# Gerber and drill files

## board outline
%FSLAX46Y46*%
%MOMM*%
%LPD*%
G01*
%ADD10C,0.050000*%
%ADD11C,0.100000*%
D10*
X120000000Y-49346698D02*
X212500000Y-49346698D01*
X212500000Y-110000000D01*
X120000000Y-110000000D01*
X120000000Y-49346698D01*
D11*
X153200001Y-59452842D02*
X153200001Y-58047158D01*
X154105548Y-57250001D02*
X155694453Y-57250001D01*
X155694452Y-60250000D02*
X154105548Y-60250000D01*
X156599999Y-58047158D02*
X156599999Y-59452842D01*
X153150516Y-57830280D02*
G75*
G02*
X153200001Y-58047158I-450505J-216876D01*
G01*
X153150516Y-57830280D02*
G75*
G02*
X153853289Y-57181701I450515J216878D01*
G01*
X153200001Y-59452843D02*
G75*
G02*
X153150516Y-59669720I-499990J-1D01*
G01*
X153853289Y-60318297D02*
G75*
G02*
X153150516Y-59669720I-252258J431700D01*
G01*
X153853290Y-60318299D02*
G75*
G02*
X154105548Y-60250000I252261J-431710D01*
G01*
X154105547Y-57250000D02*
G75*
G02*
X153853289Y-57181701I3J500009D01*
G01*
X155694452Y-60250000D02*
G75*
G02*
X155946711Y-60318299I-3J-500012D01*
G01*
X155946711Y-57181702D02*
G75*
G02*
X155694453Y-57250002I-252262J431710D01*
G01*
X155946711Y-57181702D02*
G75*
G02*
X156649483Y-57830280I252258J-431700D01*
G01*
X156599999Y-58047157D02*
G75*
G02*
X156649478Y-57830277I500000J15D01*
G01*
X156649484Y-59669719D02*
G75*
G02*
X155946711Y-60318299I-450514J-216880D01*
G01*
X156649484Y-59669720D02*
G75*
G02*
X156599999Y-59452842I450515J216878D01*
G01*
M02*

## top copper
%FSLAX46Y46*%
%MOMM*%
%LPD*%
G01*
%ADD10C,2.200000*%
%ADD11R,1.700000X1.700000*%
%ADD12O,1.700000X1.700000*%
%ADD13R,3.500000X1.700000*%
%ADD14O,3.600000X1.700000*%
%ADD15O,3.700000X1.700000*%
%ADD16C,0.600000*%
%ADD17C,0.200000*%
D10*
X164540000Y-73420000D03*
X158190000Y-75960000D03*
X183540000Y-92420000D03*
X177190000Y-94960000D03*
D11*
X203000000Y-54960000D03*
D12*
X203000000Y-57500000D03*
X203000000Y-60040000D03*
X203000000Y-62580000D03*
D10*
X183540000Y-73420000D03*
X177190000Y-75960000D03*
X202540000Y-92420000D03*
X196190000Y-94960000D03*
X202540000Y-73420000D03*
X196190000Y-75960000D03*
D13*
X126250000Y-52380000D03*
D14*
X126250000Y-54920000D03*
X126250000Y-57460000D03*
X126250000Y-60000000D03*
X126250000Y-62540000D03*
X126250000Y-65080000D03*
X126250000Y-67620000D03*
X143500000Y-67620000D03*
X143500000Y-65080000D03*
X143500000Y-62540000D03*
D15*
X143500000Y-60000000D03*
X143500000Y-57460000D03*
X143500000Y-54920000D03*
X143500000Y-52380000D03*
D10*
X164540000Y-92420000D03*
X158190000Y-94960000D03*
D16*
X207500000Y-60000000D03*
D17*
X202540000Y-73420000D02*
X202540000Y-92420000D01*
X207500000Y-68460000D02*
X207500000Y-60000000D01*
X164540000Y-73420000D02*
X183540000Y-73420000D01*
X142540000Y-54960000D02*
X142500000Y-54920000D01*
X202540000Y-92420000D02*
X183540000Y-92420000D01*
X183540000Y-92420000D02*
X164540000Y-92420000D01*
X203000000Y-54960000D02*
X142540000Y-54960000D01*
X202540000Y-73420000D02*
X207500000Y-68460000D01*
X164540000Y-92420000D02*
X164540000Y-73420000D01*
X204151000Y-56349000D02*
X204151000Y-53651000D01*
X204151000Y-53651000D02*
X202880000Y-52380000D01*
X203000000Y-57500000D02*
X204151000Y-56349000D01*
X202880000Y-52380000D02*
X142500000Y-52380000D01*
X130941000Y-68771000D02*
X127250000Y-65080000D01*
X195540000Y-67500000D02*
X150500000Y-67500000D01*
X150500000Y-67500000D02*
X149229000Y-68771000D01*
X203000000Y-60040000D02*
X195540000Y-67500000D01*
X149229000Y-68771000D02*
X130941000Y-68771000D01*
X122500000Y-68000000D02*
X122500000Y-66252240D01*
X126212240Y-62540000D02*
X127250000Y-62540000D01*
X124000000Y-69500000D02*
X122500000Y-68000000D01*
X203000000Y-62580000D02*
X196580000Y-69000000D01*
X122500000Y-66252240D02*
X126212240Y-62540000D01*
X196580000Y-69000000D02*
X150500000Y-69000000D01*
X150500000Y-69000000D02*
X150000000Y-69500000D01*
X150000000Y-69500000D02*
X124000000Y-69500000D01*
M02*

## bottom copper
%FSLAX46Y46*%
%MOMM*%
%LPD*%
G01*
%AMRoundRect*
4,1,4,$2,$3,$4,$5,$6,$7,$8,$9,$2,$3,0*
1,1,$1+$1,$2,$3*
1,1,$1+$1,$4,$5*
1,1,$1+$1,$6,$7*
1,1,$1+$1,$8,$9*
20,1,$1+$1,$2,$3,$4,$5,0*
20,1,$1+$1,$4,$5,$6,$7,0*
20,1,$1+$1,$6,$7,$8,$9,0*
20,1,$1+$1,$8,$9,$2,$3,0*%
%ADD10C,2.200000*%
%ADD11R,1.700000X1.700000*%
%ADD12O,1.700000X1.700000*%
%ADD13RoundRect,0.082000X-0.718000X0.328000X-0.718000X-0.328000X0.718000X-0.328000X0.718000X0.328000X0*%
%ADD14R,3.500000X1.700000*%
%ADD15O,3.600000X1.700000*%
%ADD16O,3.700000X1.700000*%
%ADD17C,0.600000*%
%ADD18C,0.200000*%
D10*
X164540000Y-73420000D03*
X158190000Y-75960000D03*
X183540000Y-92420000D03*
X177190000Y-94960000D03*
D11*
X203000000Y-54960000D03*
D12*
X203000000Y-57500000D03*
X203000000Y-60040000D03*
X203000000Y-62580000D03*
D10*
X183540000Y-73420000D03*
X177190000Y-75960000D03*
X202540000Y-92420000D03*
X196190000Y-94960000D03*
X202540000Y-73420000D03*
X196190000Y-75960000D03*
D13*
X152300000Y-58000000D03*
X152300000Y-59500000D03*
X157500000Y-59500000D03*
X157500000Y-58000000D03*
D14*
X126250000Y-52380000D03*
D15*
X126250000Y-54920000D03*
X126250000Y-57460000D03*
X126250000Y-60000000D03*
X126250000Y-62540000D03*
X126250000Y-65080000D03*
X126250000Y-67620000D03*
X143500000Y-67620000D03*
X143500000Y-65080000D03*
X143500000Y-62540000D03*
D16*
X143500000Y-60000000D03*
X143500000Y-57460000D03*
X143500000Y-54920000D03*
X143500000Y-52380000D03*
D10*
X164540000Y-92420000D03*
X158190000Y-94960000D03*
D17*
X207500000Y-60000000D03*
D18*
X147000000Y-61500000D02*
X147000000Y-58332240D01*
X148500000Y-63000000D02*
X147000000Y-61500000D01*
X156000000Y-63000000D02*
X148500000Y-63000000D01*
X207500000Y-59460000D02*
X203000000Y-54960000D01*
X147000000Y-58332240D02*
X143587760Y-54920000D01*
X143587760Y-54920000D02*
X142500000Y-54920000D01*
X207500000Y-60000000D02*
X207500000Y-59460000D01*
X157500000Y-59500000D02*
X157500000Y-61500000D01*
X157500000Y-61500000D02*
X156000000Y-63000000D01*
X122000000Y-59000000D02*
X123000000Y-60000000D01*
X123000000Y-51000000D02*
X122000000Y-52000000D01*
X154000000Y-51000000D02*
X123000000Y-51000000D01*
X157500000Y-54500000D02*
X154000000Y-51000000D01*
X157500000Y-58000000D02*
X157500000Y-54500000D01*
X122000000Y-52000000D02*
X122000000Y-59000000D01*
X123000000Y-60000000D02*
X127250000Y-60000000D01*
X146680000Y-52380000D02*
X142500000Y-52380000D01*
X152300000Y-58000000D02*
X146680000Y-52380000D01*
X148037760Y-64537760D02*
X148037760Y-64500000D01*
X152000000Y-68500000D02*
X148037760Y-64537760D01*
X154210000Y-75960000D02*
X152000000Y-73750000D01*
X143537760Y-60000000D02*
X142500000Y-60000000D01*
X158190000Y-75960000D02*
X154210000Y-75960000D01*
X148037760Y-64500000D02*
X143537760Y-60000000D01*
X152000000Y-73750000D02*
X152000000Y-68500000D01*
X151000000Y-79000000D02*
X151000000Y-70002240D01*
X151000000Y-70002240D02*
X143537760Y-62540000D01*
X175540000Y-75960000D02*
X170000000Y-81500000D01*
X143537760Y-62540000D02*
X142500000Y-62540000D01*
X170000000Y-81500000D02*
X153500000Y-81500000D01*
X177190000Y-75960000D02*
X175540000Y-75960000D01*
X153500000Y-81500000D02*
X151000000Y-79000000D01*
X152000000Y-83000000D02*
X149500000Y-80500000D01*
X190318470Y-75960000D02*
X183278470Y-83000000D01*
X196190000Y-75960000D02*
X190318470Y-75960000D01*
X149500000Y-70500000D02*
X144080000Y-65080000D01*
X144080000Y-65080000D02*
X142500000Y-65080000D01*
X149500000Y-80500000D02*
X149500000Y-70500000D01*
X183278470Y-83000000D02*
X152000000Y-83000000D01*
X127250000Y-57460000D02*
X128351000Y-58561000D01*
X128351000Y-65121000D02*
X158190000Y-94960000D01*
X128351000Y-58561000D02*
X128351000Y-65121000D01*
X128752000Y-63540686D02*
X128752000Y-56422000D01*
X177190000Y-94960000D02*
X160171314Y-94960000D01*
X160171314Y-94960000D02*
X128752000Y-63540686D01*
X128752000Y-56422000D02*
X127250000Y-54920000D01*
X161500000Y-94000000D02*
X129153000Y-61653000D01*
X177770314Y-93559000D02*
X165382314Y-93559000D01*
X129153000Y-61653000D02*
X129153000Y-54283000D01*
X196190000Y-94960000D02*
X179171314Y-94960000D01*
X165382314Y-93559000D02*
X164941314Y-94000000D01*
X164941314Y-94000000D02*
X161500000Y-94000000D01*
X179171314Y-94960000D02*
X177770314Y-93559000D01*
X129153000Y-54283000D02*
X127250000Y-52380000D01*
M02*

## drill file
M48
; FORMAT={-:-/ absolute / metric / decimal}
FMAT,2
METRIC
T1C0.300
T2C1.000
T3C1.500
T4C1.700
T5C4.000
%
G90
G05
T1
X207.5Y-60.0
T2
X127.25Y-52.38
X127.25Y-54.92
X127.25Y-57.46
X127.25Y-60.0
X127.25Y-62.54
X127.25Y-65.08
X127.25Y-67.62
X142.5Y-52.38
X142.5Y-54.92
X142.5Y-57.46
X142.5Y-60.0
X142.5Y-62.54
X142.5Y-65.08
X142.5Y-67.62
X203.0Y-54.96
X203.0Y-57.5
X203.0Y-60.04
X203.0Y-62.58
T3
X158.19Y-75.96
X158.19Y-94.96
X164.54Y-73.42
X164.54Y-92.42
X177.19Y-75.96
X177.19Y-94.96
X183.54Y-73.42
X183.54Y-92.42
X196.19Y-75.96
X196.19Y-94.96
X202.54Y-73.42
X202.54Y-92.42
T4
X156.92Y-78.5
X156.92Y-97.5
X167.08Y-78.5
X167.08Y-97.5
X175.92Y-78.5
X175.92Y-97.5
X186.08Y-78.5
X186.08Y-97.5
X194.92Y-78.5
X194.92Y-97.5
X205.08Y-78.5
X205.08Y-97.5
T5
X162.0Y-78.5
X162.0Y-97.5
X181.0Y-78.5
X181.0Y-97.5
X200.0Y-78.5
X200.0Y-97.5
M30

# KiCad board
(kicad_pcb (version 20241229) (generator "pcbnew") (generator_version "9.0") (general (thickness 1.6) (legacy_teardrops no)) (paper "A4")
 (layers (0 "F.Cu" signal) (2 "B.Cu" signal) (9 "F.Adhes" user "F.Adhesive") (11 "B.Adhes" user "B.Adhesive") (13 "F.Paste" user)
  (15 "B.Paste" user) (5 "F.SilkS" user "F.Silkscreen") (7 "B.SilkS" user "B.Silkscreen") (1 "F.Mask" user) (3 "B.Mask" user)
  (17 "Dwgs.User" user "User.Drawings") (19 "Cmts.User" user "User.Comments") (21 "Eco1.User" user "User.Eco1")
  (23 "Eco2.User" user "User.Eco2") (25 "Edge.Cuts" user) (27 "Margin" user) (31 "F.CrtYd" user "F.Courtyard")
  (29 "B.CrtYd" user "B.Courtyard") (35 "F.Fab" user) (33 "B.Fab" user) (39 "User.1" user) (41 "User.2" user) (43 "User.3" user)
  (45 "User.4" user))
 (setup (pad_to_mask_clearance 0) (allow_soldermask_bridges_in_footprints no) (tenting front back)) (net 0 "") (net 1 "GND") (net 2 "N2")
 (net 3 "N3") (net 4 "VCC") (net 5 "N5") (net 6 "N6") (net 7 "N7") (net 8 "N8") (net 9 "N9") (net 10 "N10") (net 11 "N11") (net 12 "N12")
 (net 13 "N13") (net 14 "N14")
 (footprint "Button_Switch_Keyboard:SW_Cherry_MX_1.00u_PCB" (layer "F.Cu") (at 164.54 73.42)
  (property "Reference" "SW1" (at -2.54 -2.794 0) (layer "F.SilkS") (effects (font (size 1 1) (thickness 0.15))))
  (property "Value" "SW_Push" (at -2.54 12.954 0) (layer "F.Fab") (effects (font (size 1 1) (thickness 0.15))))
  (pad "" np_thru_hole circle (at -7.62 5.08) (size 1.7 1.7) (drill 1.7) (layers "*.Cu" "*.Mask"))
  (pad "" np_thru_hole circle (at -2.54 5.08) (size 4 4) (drill 4) (layers "*.Cu" "*.Mask"))
  (pad "" np_thru_hole circle (at 2.54 5.08) (size 1.7 1.7) (drill 1.7) (layers "*.Cu" "*.Mask"))
  (pad "1" thru_hole circle (at 0 0) (size 2.2 2.2) (drill 1.5) (layers "*.Cu" "*.Mask") (remove_unused_layers no) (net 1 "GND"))
  (pad "2" thru_hole circle (at -6.35 2.54) (size 2.2 2.2) (drill 1.5) (layers "*.Cu" "*.Mask") (remove_unused_layers no) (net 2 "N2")))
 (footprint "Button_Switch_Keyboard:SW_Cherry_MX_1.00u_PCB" (layer "F.Cu") (at 183.54 92.42)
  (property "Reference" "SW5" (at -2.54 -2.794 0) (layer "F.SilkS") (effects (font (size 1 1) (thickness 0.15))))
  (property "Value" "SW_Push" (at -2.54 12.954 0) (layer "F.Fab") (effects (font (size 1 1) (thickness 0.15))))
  (pad "" np_thru_hole circle (at -7.62 5.08) (size 1.7 1.7) (drill 1.7) (layers "*.Cu" "*.Mask"))
  (pad "" np_thru_hole circle (at -2.54 5.08) (size 4 4) (drill 4) (layers "*.Cu" "*.Mask"))
  (pad "" np_thru_hole circle (at 2.54 5.08) (size 1.7 1.7) (drill 1.7) (layers "*.Cu" "*.Mask"))
  (pad "1" thru_hole circle (at 0 0) (size 2.2 2.2) (drill 1.5) (layers "*.Cu" "*.Mask") (remove_unused_layers no) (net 1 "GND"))
  (pad "2" thru_hole circle (at -6.35 2.54) (size 2.2 2.2) (drill 1.5) (layers "*.Cu" "*.Mask") (remove_unused_layers no) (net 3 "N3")))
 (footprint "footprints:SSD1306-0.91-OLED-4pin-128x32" (layer "F.Cu") (at 166.5 52.77)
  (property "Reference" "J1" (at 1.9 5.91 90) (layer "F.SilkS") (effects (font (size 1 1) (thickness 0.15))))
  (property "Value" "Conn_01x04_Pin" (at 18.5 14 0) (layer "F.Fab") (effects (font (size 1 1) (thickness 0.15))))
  (pad "1" thru_hole rect (at 36.5 2.19) (size 1.7 1.7) (drill 1) (layers "*.Cu" "*.Mask") (remove_unused_layers no) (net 1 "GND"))
  (pad "2" thru_hole oval (at 36.5 4.73) (size 1.7 1.7) (drill 1) (layers "*.Cu" "*.Mask") (remove_unused_layers no) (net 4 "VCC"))
  (pad "3" thru_hole oval (at 36.5 7.27) (size 1.7 1.7) (drill 1) (layers "*.Cu" "*.Mask") (remove_unused_layers no) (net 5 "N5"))
  (pad "4" thru_hole oval (at 36.5 9.81) (size 1.7 1.7) (drill 1) (layers "*.Cu" "*.Mask") (remove_unused_layers no) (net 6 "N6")))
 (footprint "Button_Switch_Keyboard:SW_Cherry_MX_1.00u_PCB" (layer "F.Cu") (at 183.54 73.42)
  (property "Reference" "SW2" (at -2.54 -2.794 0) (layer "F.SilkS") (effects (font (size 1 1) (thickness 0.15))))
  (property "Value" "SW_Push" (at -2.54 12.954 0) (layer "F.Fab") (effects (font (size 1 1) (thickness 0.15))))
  (pad "" np_thru_hole circle (at -7.62 5.08) (size 1.7 1.7) (drill 1.7) (layers "*.Cu" "*.Mask"))
  (pad "" np_thru_hole circle (at -2.54 5.08) (size 4 4) (drill 4) (layers "*.Cu" "*.Mask"))
  (pad "" np_thru_hole circle (at 2.54 5.08) (size 1.7 1.7) (drill 1.7) (layers "*.Cu" "*.Mask"))
  (pad "1" thru_hole circle (at 0 0) (size 2.2 2.2) (drill 1.5) (layers "*.Cu" "*.Mask") (remove_unused_layers no) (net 1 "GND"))
  (pad "2" thru_hole circle (at -6.35 2.54) (size 2.2 2.2) (drill 1.5) (layers "*.Cu" "*.Mask") (remove_unused_layers no) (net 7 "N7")))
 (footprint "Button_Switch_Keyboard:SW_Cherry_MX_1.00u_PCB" (layer "F.Cu") (at 202.54 92.42)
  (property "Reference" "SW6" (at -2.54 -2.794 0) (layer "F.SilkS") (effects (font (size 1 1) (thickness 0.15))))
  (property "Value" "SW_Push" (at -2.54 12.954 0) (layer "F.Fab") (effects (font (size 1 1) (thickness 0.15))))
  (pad "" np_thru_hole circle (at -7.62 5.08) (size 1.7 1.7) (drill 1.7) (layers "*.Cu" "*.Mask"))
  (pad "" np_thru_hole circle (at -2.54 5.08) (size 4 4) (drill 4) (layers "*.Cu" "*.Mask"))
  (pad "" np_thru_hole circle (at 2.54 5.08) (size 1.7 1.7) (drill 1.7) (layers "*.Cu" "*.Mask"))
  (pad "1" thru_hole circle (at 0 0) (size 2.2 2.2) (drill 1.5) (layers "*.Cu" "*.Mask") (remove_unused_layers no) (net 1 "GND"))
  (pad "2" thru_hole circle (at -6.35 2.54) (size 2.2 2.2) (drill 1.5) (layers "*.Cu" "*.Mask") (remove_unused_layers no) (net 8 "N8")))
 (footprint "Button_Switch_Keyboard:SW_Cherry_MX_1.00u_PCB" (layer "F.Cu") (at 202.54 73.42)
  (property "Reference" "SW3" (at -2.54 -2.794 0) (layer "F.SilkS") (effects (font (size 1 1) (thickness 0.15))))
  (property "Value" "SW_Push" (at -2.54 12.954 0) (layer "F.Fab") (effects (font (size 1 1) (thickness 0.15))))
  (pad "" np_thru_hole circle (at -7.62 5.08) (size 1.7 1.7) (drill 1.7) (layers "*.Cu" "*.Mask"))
  (pad "" np_thru_hole circle (at -2.54 5.08) (size 4 4) (drill 4) (layers "*.Cu" "*.Mask"))
  (pad "" np_thru_hole circle (at 2.54 5.08) (size 1.7 1.7) (drill 1.7) (layers "*.Cu" "*.Mask"))
  (pad "1" thru_hole circle (at 0 0) (size 2.2 2.2) (drill 1.5) (layers "*.Cu" "*.Mask") (remove_unused_layers no) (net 1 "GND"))
  (pad "2" thru_hole circle (at -6.35 2.54) (size 2.2 2.2) (drill 1.5) (layers "*.Cu" "*.Mask") (remove_unused_layers no) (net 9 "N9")))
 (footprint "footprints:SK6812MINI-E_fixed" (layer "F.Cu") (at 154.899999 58.852842)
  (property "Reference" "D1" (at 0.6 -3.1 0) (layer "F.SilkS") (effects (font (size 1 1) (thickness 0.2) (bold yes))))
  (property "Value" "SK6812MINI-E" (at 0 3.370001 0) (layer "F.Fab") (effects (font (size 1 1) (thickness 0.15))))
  (fp_line (start -1.699998 0.6) (end -1.699998 -0.805684) (stroke (width 0.1) (type solid)) (layer "Edge.Cuts"))
  (fp_line (start -0.794451 -1.602841) (end 0.794454 -1.602841) (stroke (width 0.1) (type solid)) (layer "Edge.Cuts"))
  (fp_line (start 0.794453 1.397158) (end -0.794451 1.397158) (stroke (width 0.1) (type solid)) (layer "Edge.Cuts"))
  (fp_line (start 1.7 -0.805684) (end 1.7 0.6) (stroke (width 0.1) (type solid)) (layer "Edge.Cuts"))
  (fp_arc (start -1.749483 -1.022562) (mid -1.712526 -0.91691) (end -1.699998 -0.805684) (stroke (width 0.1) (type solid))
   (layer "Edge.Cuts"))
  (fp_arc (start -1.749483 -1.022562) (mid -1.63807 -1.606877) (end -1.04671 -1.671141) (stroke (width 0.1) (type solid))
   (layer "Edge.Cuts"))
  (fp_arc (start -1.699998 0.600001) (mid -1.712526 0.711226) (end -1.749483 0.816878) (stroke (width 0.1) (type solid)) (layer "Edge.Cuts"))
  (fp_arc (start -1.04671 1.465455) (mid -1.638069 1.401192) (end -1.749483 0.816878) (stroke (width 0.1) (type solid)) (layer "Edge.Cuts"))
  (fp_arc (start -1.046709 1.465457) (mid -0.925121 1.414535) (end -0.794451 1.397158) (stroke (width 0.1) (type solid)) (layer "Edge.Cuts"))
  (fp_arc (start -0.794452 -1.602842) (mid -0.925122 -1.620219) (end -1.04671 -1.671141) (stroke (width 0.1) (type solid))
   (layer "Edge.Cuts"))
  (fp_arc (start 0.794453 1.397158) (mid 0.925124 1.414535) (end 1.046712 1.465457) (stroke (width 0.1) (type solid)) (layer "Edge.Cuts"))
  (fp_arc (start 1.046712 -1.67114) (mid 0.925124 -1.620218) (end 0.794454 -1.602841) (stroke (width 0.1) (type solid)) (layer "Edge.Cuts"))
  (fp_arc (start 1.046712 -1.67114) (mid 1.638072 -1.606876) (end 1.749485 -1.022562) (stroke (width 0.1) (type solid)) (layer "Edge.Cuts"))
  (fp_arc (start 1.7 -0.805685) (mid 1.712528 -0.91691) (end 1.749485 -1.022562) (stroke (width 0.1) (type solid)) (layer "Edge.Cuts"))
  (fp_arc (start 1.749485 0.816877) (mid 1.638073 1.401193) (end 1.046712 1.465457) (stroke (width 0.1) (type solid)) (layer "Edge.Cuts"))
  (fp_arc (start 1.749485 0.816878) (mid 1.712528 0.711226) (end 1.7 0.6) (stroke (width 0.1) (type solid)) (layer "Edge.Cuts"))
  (pad "1" smd roundrect (at -2.599999 -0.852842 270) (size 0.82 1.6) (layers "B.Cu" "B.Mask" "B.Paste") (roundrect_rratio 0.1)
   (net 4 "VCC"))
  (pad "2" smd roundrect (at -2.599999 0.647158 270) (size 0.82 1.6) (layers "B.Cu" "B.Mask" "B.Paste") (roundrect_rratio 0.1))
  (pad "3" smd roundrect (at 2.600001 0.647158 270) (size 0.82 1.6) (layers "B.Cu" "B.Mask" "B.Paste") (roundrect_rratio 0.1) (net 1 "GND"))
  (pad "4" smd roundrect (at 2.600001 -0.852842 270) (size 0.82 1.6) (layers "B.Cu" "B.Mask" "B.Paste") (roundrect_rratio 0.1)
   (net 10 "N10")))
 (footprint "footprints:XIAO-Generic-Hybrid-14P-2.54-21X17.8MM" (layer "F.Cu") (at 134.875 60)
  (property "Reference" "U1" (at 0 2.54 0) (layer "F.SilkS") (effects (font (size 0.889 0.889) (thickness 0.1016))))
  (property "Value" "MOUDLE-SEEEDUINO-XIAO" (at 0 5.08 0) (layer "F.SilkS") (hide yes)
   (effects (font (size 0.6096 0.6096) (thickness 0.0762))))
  (pad "1" thru_hole rect (at -7.625 -7.62) (size 3.5 1.7) (drill 1 (offset -1 0)) (layers "*.Cu" "*.Mask") (remove_unused_layers no)
   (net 8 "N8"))
  (pad "2" thru_hole oval (at -7.625 -5.08) (size 3.6 1.7) (drill 1 (offset -1 0)) (layers "*.Cu" "*.Mask") (remove_unused_layers no)
   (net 3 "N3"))
  (pad "3" thru_hole oval (at -7.625 -2.54) (size 3.6 1.7) (drill 1 (offset -1 0)) (layers "*.Cu" "*.Mask") (remove_unused_layers no)
   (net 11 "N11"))
  (pad "4" thru_hole oval (at -7.625 0) (size 3.6 1.7) (drill 1 (offset -1 0)) (layers "*.Cu" "*.Mask") (remove_unused_layers no)
   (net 10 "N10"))
  (pad "5" thru_hole oval (at -7.625 2.54) (size 3.6 1.7) (drill 1 (offset -1 0)) (layers "*.Cu" "*.Mask") (remove_unused_layers no)
   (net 6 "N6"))
  (pad "6" thru_hole oval (at -7.625 5.08 180) (size 3.6 1.7) (drill 1 (offset 1 0)) (layers "*.Cu" "*.Mask") (remove_unused_layers no)
   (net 5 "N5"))
  (pad "7" thru_hole oval (at -7.625 7.62) (size 3.6 1.7) (drill 1 (offset -1 0)) (layers "*.Cu" "*.Mask") (remove_unused_layers no)
   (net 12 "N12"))
  (pad "8" thru_hole oval (at 7.625 7.62) (size 3.6 1.7) (drill 1 (offset 1 0)) (layers "*.Cu" "*.Mask") (remove_unused_layers no)
   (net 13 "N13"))
  (pad "9" thru_hole oval (at 7.625 5.08) (size 3.6 1.7) (drill 1 (offset 1 0)) (layers "*.Cu" "*.Mask") (remove_unused_layers no)
   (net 9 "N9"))
  (pad "10" thru_hole oval (at 7.625 2.54) (size 3.6 1.7) (drill 1 (offset 1 0)) (layers "*.Cu" "*.Mask") (remove_unused_layers no)
   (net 7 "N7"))
  (pad "11" thru_hole oval (at 7.625 0) (size 3.7 1.7) (drill 1 (offset 1 0)) (layers "*.Cu" "*.Mask") (remove_unused_layers no)
   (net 2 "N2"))
  (pad "12" thru_hole oval (at 7.625 -2.54) (size 3.7 1.7) (drill 1 (offset 1 0)) (layers "*.Cu" "*.Mask") (remove_unused_layers no)
   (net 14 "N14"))
  (pad "13" thru_hole oval (at 7.625 -5.08) (size 3.7 1.7) (drill 1 (offset 1 0)) (layers "*.Cu" "*.Mask") (remove_unused_layers no)
   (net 1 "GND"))
  (pad "14" thru_hole oval (at 7.625 -7.62) (size 3.7 1.7) (drill 1 (offset 1 0)) (layers "*.Cu" "*.Mask") (remove_unused_layers no)
   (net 4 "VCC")))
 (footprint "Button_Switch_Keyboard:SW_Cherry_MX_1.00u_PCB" (layer "F.Cu") (at 164.54 92.42)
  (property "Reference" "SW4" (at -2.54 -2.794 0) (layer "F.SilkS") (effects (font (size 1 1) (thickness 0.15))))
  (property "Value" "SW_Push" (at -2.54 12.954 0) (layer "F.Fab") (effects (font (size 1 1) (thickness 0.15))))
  (pad "" np_thru_hole circle (at -7.62 5.08) (size 1.7 1.7) (drill 1.7) (layers "*.Cu" "*.Mask"))
  (pad "" np_thru_hole circle (at -2.54 5.08) (size 4 4) (drill 4) (layers "*.Cu" "*.Mask"))
  (pad "" np_thru_hole circle (at 2.54 5.08) (size 1.7 1.7) (drill 1.7) (layers "*.Cu" "*.Mask"))
  (pad "1" thru_hole circle (at 0 0) (size 2.2 2.2) (drill 1.5) (layers "*.Cu" "*.Mask") (remove_unused_layers no) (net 1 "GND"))
  (pad "2" thru_hole circle (at -6.35 2.54) (size 2.2 2.2) (drill 1.5) (layers "*.Cu" "*.Mask") (remove_unused_layers no) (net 11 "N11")))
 (gr_rect (start 120 49.346698) (end 212.5 110) (stroke (width 0.05) (type default)) (fill no) (layer "Edge.Cuts"))
 (segment (start 202.54 73.42) (end 202.54 92.42) (width 0.2) (layer "F.Cu") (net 1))
 (segment (start 207.5 68.46) (end 207.5 60) (width 0.2) (layer "F.Cu") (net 1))
 (segment (start 164.54 73.42) (end 183.54 73.42) (width 0.2) (layer "F.Cu") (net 1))
 (segment (start 142.54 54.96) (end 142.5 54.92) (width 0.2) (layer "F.Cu") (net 1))
 (segment (start 202.54 92.42) (end 183.54 92.42) (width 0.2) (layer "F.Cu") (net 1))
 (segment (start 183.54 92.42) (end 164.54 92.42) (width 0.2) (layer "F.Cu") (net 1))
 (segment (start 203 54.96) (end 142.54 54.96) (width 0.2) (layer "F.Cu") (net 1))
 (segment (start 202.54 73.42) (end 207.5 68.46) (width 0.2) (layer "F.Cu") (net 1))
 (segment (start 164.54 92.42) (end 164.54 73.42) (width 0.2) (layer "F.Cu") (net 1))
 (via (at 207.5 60) (size 0.6) (drill 0.3) (layers "F.Cu" "B.Cu") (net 1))
 (segment (start 147 61.5) (end 147 58.33224) (width 0.2) (layer "B.Cu") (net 1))
 (segment (start 148.5 63) (end 147 61.5) (width 0.2) (layer "B.Cu") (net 1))
 (segment (start 156 63) (end 148.5 63) (width 0.2) (layer "B.Cu") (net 1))
 (segment (start 207.5 59.46) (end 203 54.96) (width 0.2) (layer "B.Cu") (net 1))
 (segment (start 147 58.33224) (end 143.58776 54.92) (width 0.2) (layer "B.Cu") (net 1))
 (segment (start 143.58776 54.92) (end 142.5 54.92) (width 0.2) (layer "B.Cu") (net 1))
 (segment (start 207.5 60) (end 207.5 59.46) (width 0.2) (layer "B.Cu") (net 1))
 (segment (start 157.5 59.5) (end 157.5 61.5) (width 0.2) (layer "B.Cu") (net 1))
 (segment (start 157.5 61.5) (end 156 63) (width 0.2) (layer "B.Cu") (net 1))
 (segment (start 122 59) (end 123 60) (width 0.2) (layer "B.Cu") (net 10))
 (segment (start 123 51) (end 122 52) (width 0.2) (layer "B.Cu") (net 10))
 (segment (start 154 51) (end 123 51) (width 0.2) (layer "B.Cu") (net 10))
 (segment (start 157.5 54.5) (end 154 51) (width 0.2) (layer "B.Cu") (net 10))
 (segment (start 157.5 58) (end 157.5 54.5) (width 0.2) (layer "B.Cu") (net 10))
 (segment (start 122 52) (end 122 59) (width 0.2) (layer "B.Cu") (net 10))
 (segment (start 123 60) (end 127.25 60) (width 0.2) (layer "B.Cu") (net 10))
 (segment (start 204.151 56.349) (end 204.151 53.651) (width 0.2) (layer "F.Cu") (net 4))
 (segment (start 204.151 53.651) (end 202.88 52.38) (width 0.2) (layer "F.Cu") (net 4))
 (segment (start 203 57.5) (end 204.151 56.349) (width 0.2) (layer "F.Cu") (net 4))
 (segment (start 202.88 52.38) (end 142.5 52.38) (width 0.2) (layer "F.Cu") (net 4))
 (segment (start 146.68 52.38) (end 142.5 52.38) (width 0.2) (layer "B.Cu") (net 4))
 (segment (start 152.3 58) (end 146.68 52.38) (width 0.2) (layer "B.Cu") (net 4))
 (segment (start 130.941 68.771) (end 127.25 65.08) (width 0.2) (layer "F.Cu") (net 5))
 (segment (start 195.54 67.5) (end 150.5 67.5) (width 0.2) (layer "F.Cu") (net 5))
 (segment (start 150.5 67.5) (end 149.229 68.771) (width 0.2) (layer "F.Cu") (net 5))
 (segment (start 203 60.04) (end 195.54 67.5) (width 0.2) (layer "F.Cu") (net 5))
 (segment (start 149.229 68.771) (end 130.941 68.771) (width 0.2) (layer "F.Cu") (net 5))
 (segment (start 122.5 68) (end 122.5 66.25224) (width 0.2) (layer "F.Cu") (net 6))
 (segment (start 126.21224 62.54) (end 127.25 62.54) (width 0.2) (layer "F.Cu") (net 6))
 (segment (start 124 69.5) (end 122.5 68) (width 0.2) (layer "F.Cu") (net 6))
 (segment (start 203 62.58) (end 196.58 69) (width 0.2) (layer "F.Cu") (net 6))
 (segment (start 122.5 66.25224) (end 126.21224 62.54) (width 0.2) (layer "F.Cu") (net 6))
 (segment (start 196.58 69) (end 150.5 69) (width 0.2) (layer "F.Cu") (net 6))
 (segment (start 150.5 69) (end 150 69.5) (width 0.2) (layer "F.Cu") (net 6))
 (segment (start 150 69.5) (end 124 69.5) (width 0.2) (layer "F.Cu") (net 6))
 (segment (start 148.03776 64.53776) (end 148.03776 64.5) (width 0.2) (layer "B.Cu") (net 2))
 (segment (start 152 68.5) (end 148.03776 64.53776) (width 0.2) (layer "B.Cu") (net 2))
 (segment (start 154.21 75.96) (end 152 73.75) (width 0.2) (layer "B.Cu") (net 2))
 (segment (start 143.53776 60) (end 142.5 60) (width 0.2) (layer "B.Cu") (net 2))
 (segment (start 158.19 75.96) (end 154.21 75.96) (width 0.2) (layer "B.Cu") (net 2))
 (segment (start 148.03776 64.5) (end 143.53776 60) (width 0.2) (layer "B.Cu") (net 2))
 (segment (start 152 73.75) (end 152 68.5) (width 0.2) (layer "B.Cu") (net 2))
 (segment (start 151 79) (end 151 70.00224) (width 0.2) (layer "B.Cu") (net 7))
 (segment (start 151 70.00224) (end 143.53776 62.54) (width 0.2) (layer "B.Cu") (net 7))
 (segment (start 175.54 75.96) (end 170 81.5) (width 0.2) (layer "B.Cu") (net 7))
 (segment (start 143.53776 62.54) (end 142.5 62.54) (width 0.2) (layer "B.Cu") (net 7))
 (segment (start 170 81.5) (end 153.5 81.5) (width 0.2) (layer "B.Cu") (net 7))
 (segment (start 177.19 75.96) (end 175.54 75.96) (width 0.2) (layer "B.Cu") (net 7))
 (segment (start 153.5 81.5) (end 151 79) (width 0.2) (layer "B.Cu") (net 7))
 (segment (start 152 83) (end 149.5 80.5) (width 0.2) (layer "B.Cu") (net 9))
 (segment (start 190.31847 75.96) (end 183.27847 83) (width 0.2) (layer "B.Cu") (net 9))
 (segment (start 196.19 75.96) (end 190.31847 75.96) (width 0.2) (layer "B.Cu") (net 9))
 (segment (start 149.5 70.5) (end 144.08 65.08) (width 0.2) (layer "B.Cu") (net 9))
 (segment (start 144.08 65.08) (end 142.5 65.08) (width 0.2) (layer "B.Cu") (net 9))
 (segment (start 149.5 80.5) (end 149.5 70.5) (width 0.2) (layer "B.Cu") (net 9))
 (segment (start 183.27847 83) (end 152 83) (width 0.2) (layer "B.Cu") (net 9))
 (segment (start 127.25 57.46) (end 128.351 58.561) (width 0.2) (layer "B.Cu") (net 11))
 (segment (start 128.351 65.121) (end 158.19 94.96) (width 0.2) (layer "B.Cu") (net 11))
 (segment (start 128.351 58.561) (end 128.351 65.121) (width 0.2) (layer "B.Cu") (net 11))
 (segment (start 128.752 63.540686) (end 128.752 56.422) (width 0.2) (layer "B.Cu") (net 3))
 (segment (start 177.19 94.96) (end 160.171314 94.96) (width 0.2) (layer "B.Cu") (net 3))
 (segment (start 160.171314 94.96) (end 128.752 63.540686) (width 0.2) (layer "B.Cu") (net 3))
 (segment (start 128.752 56.422) (end 127.25 54.92) (width 0.2) (layer "B.Cu") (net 3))
 (segment (start 161.5 94) (end 129.153 61.653) (width 0.2) (layer "B.Cu") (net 8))
 (segment (start 177.770314 93.559) (end 165.382314 93.559) (width 0.2) (layer "B.Cu") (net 8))
 (segment (start 129.153 61.653) (end 129.153 54.283) (width 0.2) (layer "B.Cu") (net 8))
 (segment (start 196.19 94.96) (end 179.171314 94.96) (width 0.2) (layer "B.Cu") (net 8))
 (segment (start 165.382314 93.559) (end 164.941314 94) (width 0.2) (layer "B.Cu") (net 8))
 (segment (start 164.941314 94) (end 161.5 94) (width 0.2) (layer "B.Cu") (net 8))
 (segment (start 179.171314 94.96) (end 177.770314 93.559) (width 0.2) (layer "B.Cu") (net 8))
 (segment (start 129.153 54.283) (end 127.25 52.38) (width 0.2) (layer "B.Cu") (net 8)))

